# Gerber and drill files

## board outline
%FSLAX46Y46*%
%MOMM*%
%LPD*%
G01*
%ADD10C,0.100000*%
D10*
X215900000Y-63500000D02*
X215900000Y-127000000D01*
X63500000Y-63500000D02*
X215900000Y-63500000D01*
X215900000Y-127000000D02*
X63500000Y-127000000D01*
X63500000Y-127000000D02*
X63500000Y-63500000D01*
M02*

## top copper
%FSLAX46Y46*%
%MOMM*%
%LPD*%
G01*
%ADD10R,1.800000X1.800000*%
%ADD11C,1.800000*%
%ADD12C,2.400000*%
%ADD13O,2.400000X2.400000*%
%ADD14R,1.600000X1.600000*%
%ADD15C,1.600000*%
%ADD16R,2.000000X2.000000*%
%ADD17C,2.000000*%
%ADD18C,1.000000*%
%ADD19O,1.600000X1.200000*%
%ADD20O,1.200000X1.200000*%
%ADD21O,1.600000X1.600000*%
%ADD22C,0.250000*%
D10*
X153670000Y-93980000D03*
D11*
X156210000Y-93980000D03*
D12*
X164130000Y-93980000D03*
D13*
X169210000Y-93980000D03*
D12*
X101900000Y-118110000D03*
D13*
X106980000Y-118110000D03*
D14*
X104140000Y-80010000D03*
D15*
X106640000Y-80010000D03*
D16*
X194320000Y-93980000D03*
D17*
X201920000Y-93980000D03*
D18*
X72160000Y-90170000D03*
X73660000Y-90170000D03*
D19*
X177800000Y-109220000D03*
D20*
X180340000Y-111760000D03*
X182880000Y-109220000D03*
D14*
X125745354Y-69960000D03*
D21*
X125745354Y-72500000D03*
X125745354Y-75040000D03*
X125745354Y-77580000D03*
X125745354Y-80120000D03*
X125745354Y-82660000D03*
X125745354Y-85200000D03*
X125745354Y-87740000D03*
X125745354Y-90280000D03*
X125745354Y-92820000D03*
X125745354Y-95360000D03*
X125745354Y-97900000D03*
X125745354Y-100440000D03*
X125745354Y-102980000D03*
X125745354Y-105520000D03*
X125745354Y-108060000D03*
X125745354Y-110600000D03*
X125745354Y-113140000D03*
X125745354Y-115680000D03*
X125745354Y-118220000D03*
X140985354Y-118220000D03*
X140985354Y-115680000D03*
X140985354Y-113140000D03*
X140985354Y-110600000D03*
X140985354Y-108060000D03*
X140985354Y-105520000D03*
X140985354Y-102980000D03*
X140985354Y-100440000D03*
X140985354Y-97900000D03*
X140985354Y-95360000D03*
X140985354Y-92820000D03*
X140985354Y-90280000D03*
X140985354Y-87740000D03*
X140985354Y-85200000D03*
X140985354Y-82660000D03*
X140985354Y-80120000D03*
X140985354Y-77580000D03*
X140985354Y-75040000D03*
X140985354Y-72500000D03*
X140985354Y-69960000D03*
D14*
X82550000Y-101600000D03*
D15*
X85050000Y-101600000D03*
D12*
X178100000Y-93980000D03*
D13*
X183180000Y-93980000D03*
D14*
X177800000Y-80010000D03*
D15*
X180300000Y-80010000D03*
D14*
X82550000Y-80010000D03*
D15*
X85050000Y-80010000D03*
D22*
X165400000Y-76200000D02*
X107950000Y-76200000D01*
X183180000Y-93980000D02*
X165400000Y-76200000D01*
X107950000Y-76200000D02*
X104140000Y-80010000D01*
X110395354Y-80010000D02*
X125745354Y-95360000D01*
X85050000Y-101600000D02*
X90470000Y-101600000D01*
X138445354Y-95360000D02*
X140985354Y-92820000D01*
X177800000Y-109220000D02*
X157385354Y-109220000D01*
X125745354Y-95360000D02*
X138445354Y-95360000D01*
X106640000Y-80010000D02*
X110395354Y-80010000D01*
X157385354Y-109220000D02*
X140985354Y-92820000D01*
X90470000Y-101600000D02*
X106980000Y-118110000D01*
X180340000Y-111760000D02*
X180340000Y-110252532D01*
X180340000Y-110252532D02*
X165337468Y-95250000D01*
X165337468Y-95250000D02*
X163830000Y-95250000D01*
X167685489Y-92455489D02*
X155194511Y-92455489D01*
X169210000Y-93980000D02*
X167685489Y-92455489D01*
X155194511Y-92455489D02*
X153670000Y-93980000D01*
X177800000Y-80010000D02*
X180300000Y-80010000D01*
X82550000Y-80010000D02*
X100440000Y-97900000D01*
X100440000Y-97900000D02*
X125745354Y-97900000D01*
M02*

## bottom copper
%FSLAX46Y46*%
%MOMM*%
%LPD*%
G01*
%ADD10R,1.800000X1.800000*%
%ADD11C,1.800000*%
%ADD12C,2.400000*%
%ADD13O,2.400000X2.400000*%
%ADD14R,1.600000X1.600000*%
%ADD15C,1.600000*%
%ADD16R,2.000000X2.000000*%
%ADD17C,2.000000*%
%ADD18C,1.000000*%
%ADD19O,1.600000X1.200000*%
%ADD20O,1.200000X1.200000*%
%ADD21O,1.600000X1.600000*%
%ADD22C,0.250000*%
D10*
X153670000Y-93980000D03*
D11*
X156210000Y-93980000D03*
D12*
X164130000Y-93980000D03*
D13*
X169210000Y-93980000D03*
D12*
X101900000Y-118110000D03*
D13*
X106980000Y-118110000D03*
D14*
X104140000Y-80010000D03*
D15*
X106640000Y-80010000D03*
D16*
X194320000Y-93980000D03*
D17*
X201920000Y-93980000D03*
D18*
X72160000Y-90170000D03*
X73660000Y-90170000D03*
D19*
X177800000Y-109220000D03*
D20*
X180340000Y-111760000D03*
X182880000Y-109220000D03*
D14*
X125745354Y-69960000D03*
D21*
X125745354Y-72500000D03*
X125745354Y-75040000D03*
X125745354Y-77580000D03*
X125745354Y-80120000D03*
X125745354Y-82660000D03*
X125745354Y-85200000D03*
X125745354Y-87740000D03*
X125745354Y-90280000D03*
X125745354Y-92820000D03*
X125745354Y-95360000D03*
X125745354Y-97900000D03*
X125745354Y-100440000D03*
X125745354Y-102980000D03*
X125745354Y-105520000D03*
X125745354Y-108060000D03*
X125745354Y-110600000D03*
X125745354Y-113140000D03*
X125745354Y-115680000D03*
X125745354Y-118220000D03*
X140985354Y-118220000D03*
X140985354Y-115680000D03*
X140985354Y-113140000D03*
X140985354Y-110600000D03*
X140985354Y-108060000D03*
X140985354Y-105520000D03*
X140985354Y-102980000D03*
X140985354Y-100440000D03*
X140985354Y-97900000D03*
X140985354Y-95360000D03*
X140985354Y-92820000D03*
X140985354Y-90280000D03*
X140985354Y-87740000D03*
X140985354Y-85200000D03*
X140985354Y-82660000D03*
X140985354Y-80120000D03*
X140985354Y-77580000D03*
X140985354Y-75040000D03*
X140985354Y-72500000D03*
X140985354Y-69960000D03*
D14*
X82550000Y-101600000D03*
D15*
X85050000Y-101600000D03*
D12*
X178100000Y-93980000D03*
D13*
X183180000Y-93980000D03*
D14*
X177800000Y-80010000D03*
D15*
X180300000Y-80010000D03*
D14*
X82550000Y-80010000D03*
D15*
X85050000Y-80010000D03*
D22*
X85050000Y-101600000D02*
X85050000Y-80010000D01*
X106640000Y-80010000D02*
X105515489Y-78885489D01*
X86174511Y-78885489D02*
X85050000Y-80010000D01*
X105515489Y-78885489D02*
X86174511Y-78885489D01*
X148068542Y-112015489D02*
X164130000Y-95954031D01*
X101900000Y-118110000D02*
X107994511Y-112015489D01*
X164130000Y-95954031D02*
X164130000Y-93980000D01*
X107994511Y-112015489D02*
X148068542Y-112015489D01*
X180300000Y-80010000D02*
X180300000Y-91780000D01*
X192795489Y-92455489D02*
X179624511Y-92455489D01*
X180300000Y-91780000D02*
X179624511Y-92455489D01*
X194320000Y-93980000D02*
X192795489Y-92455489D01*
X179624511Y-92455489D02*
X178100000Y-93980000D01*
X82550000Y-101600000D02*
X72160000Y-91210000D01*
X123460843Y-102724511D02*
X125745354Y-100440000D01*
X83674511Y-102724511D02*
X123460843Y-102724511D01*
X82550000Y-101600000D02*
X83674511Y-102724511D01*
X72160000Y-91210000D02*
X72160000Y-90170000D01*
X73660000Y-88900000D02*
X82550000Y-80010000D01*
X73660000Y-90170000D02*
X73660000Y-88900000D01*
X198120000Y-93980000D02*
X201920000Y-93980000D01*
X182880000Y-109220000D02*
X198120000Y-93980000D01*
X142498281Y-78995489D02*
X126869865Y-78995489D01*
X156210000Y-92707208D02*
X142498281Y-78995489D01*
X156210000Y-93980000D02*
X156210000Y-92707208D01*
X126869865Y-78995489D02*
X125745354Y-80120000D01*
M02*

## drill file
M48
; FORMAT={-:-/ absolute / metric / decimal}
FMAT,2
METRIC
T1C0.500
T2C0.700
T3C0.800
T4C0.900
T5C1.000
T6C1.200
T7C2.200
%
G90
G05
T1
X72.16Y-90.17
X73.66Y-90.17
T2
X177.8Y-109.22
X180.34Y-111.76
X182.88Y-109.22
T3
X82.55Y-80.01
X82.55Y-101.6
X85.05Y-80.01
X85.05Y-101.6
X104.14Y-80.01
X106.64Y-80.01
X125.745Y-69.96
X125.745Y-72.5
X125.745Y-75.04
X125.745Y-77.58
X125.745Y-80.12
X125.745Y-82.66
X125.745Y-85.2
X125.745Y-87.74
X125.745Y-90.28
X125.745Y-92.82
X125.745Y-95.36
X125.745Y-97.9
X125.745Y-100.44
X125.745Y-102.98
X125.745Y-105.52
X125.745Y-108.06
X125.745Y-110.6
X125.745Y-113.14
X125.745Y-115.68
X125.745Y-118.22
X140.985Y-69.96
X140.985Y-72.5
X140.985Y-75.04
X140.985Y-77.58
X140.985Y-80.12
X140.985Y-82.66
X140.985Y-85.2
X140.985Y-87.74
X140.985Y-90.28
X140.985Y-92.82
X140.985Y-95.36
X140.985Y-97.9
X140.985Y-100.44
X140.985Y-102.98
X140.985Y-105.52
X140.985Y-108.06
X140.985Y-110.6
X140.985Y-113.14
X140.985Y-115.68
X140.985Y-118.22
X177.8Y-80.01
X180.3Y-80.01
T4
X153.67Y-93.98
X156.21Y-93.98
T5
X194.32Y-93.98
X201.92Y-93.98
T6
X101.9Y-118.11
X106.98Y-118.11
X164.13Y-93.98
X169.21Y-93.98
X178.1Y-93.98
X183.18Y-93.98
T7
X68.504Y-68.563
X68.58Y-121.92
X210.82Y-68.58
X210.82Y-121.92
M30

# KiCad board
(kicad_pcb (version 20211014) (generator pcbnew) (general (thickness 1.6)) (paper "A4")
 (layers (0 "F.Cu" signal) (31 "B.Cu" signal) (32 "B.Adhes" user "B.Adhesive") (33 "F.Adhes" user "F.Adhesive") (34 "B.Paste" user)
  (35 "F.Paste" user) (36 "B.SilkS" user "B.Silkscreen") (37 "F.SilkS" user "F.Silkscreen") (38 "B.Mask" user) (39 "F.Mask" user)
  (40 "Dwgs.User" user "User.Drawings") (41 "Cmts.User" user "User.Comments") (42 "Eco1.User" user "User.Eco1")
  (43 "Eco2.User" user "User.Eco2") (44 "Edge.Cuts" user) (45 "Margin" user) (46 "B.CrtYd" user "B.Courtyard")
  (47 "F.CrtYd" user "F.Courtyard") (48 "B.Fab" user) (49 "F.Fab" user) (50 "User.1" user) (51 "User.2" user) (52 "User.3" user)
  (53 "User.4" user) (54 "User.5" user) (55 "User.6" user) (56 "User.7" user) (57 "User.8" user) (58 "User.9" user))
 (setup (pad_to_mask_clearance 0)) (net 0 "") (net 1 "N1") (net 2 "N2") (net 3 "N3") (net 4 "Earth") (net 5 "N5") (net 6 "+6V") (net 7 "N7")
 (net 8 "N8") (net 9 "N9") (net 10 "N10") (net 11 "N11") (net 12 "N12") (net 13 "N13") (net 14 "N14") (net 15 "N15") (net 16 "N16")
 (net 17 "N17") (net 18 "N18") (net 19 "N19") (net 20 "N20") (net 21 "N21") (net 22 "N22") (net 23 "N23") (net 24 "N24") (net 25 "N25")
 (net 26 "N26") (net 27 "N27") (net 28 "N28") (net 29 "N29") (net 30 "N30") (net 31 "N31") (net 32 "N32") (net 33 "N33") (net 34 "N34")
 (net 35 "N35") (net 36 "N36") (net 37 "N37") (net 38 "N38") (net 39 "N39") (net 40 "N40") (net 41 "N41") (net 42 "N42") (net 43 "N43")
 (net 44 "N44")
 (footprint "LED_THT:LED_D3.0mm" (layer "F.Cu") (at 153.67 93.98)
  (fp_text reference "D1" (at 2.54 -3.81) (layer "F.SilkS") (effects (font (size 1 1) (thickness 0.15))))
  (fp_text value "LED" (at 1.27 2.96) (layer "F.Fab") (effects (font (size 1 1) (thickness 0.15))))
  (pad "1" thru_hole rect (at 0 0) (size 1.8 1.8) (drill 0.9) (layers *.Cu *.Mask) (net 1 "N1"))
  (pad "2" thru_hole circle (at 2.54 0) (size 1.8 1.8) (drill 0.9) (layers *.Cu *.Mask) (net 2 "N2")))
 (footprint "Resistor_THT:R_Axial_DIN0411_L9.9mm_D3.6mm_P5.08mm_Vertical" (layer "F.Cu") (at 164.13 93.98)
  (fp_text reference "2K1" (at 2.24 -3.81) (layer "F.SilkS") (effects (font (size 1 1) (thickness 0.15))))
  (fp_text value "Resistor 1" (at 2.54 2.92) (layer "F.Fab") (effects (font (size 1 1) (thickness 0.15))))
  (pad "1" thru_hole circle (at 0 0) (size 2.4 2.4) (drill 1.2) (layers *.Cu *.Mask) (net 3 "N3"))
  (pad "2" thru_hole oval (at 5.08 0) (size 2.4 2.4) (drill 1.2) (layers *.Cu *.Mask) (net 1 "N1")))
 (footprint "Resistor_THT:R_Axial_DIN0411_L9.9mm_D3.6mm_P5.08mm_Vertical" (layer "F.Cu") (at 101.9 118.11)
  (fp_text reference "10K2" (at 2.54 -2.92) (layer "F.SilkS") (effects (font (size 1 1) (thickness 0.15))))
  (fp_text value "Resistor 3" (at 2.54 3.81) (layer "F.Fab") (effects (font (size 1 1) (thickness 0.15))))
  (pad "1" thru_hole circle (at 0 0) (size 2.4 2.4) (drill 1.2) (layers *.Cu *.Mask) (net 3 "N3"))
  (pad "2" thru_hole oval (at 5.08 0) (size 2.4 2.4) (drill 1.2) (layers *.Cu *.Mask) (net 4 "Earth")))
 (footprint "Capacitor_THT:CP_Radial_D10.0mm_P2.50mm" (layer "F.Cu") (at 104.14 80.01)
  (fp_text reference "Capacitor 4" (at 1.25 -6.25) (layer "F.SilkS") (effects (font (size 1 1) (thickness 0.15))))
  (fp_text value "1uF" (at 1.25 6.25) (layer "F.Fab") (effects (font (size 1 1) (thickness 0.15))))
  (pad "1" thru_hole rect (at 0 0) (size 1.6 1.6) (drill 0.8) (layers *.Cu *.Mask) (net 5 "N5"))
  (pad "2" thru_hole circle (at 2.5 0) (size 1.6 1.6) (drill 0.8) (layers *.Cu *.Mask) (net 4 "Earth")))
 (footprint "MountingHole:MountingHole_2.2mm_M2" (layer "F.Cu") (at 210.82 121.92)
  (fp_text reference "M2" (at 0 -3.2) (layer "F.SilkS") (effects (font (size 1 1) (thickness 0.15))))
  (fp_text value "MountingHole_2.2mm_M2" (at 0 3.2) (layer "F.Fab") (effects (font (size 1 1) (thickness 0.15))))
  (pad "" np_thru_hole circle (at 0 0) (size 2.2 2.2) (drill 2.2) (layers *.Cu *.Mask)))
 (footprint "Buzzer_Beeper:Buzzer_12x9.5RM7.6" (layer "F.Cu") (at 194.32 93.98)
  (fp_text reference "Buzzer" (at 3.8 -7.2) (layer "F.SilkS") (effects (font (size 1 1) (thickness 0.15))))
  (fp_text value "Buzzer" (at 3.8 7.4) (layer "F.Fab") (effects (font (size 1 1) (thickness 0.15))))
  (pad "1" thru_hole rect (at 0 0) (size 2 2) (drill 1) (layers *.Cu *.Mask) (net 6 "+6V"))
  (pad "2" thru_hole circle (at 7.6 0) (size 2 2) (drill 1) (layers *.Cu *.Mask) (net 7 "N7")))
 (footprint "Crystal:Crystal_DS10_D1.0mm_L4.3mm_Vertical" (layer "F.Cu") (at 72.16 90.17)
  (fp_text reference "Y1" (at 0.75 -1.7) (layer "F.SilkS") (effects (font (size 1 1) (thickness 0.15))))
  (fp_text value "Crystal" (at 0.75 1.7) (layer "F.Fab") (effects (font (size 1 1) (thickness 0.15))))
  (pad "1" thru_hole circle (at 0 0) (size 1 1) (drill 0.5) (layers *.Cu *.Mask) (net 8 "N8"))
  (pad "2" thru_hole circle (at 1.5 0) (size 1 1) (drill 0.5) (layers *.Cu *.Mask) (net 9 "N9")))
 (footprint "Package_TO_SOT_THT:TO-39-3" (layer "F.Cu") (at 177.8 109.22)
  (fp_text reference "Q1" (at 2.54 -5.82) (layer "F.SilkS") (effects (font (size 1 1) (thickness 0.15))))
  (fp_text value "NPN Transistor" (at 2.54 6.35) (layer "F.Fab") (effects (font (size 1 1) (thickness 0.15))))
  (pad "1" thru_hole oval (at 0 0) (size 1.6 1.2) (drill 0.7) (layers *.Cu *.Mask) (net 4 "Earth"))
  (pad "2" thru_hole oval (at 2.54 2.54) (size 1.2 1.2) (drill 0.7) (layers *.Cu *.Mask) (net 3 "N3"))
  (pad "3" thru_hole oval (at 5.08 0) (size 1.2 1.2) (drill 0.7) (layers *.Cu *.Mask) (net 7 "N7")))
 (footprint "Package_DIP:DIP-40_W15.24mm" (layer "F.Cu") (at 125.745354 69.96)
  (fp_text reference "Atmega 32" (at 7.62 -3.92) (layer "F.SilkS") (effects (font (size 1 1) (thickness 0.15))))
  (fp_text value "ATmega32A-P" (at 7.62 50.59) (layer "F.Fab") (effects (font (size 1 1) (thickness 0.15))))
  (pad "1" thru_hole rect (at 0 0) (size 1.6 1.6) (drill 0.8) (layers *.Cu *.Mask) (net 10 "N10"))
  (pad "2" thru_hole oval (at 0 2.54) (size 1.6 1.6) (drill 0.8) (layers *.Cu *.Mask) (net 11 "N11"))
  (pad "3" thru_hole oval (at 0 5.08) (size 1.6 1.6) (drill 0.8) (layers *.Cu *.Mask) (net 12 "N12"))
  (pad "4" thru_hole oval (at 0 7.62) (size 1.6 1.6) (drill 0.8) (layers *.Cu *.Mask) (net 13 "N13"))
  (pad "5" thru_hole oval (at 0 10.16) (size 1.6 1.6) (drill 0.8) (layers *.Cu *.Mask) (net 2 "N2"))
  (pad "6" thru_hole oval (at 0 12.7) (size 1.6 1.6) (drill 0.8) (layers *.Cu *.Mask) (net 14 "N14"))
  (pad "7" thru_hole oval (at 0 15.24) (size 1.6 1.6) (drill 0.8) (layers *.Cu *.Mask) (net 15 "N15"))
  (pad "8" thru_hole oval (at 0 17.78) (size 1.6 1.6) (drill 0.8) (layers *.Cu *.Mask) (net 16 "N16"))
  (pad "9" thru_hole oval (at 0 20.32) (size 1.6 1.6) (drill 0.8) (layers *.Cu *.Mask) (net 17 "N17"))
  (pad "10" thru_hole oval (at 0 22.86) (size 1.6 1.6) (drill 0.8) (layers *.Cu *.Mask) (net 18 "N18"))
  (pad "11" thru_hole oval (at 0 25.4) (size 1.6 1.6) (drill 0.8) (layers *.Cu *.Mask) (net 4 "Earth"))
  (pad "12" thru_hole oval (at 0 27.94) (size 1.6 1.6) (drill 0.8) (layers *.Cu *.Mask) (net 9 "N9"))
  (pad "13" thru_hole oval (at 0 30.48) (size 1.6 1.6) (drill 0.8) (layers *.Cu *.Mask) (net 8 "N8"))
  (pad "14" thru_hole oval (at 0 33.02) (size 1.6 1.6) (drill 0.8) (layers *.Cu *.Mask) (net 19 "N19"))
  (pad "15" thru_hole oval (at 0 35.56) (size 1.6 1.6) (drill 0.8) (layers *.Cu *.Mask) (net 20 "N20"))
  (pad "16" thru_hole oval (at 0 38.1) (size 1.6 1.6) (drill 0.8) (layers *.Cu *.Mask) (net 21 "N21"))
  (pad "17" thru_hole oval (at 0 40.64) (size 1.6 1.6) (drill 0.8) (layers *.Cu *.Mask) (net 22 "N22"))
  (pad "18" thru_hole oval (at 0 43.18) (size 1.6 1.6) (drill 0.8) (layers *.Cu *.Mask) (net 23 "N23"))
  (pad "19" thru_hole oval (at 0 45.72) (size 1.6 1.6) (drill 0.8) (layers *.Cu *.Mask) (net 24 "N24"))
  (pad "20" thru_hole oval (at 0 48.26) (size 1.6 1.6) (drill 0.8) (layers *.Cu *.Mask) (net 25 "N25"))
  (pad "21" thru_hole oval (at 15.24 48.26) (size 1.6 1.6) (drill 0.8) (layers *.Cu *.Mask) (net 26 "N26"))
  (pad "22" thru_hole oval (at 15.24 45.72) (size 1.6 1.6) (drill 0.8) (layers *.Cu *.Mask) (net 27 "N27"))
  (pad "23" thru_hole oval (at 15.24 43.18) (size 1.6 1.6) (drill 0.8) (layers *.Cu *.Mask) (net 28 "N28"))
  (pad "24" thru_hole oval (at 15.24 40.64) (size 1.6 1.6) (drill 0.8) (layers *.Cu *.Mask) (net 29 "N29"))
  (pad "25" thru_hole oval (at 15.24 38.1) (size 1.6 1.6) (drill 0.8) (layers *.Cu *.Mask) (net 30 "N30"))
  (pad "26" thru_hole oval (at 15.24 35.56) (size 1.6 1.6) (drill 0.8) (layers *.Cu *.Mask) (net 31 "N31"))
  (pad "27" thru_hole oval (at 15.24 33.02) (size 1.6 1.6) (drill 0.8) (layers *.Cu *.Mask) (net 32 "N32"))
  (pad "28" thru_hole oval (at 15.24 30.48) (size 1.6 1.6) (drill 0.8) (layers *.Cu *.Mask) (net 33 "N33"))
  (pad "29" thru_hole oval (at 15.24 27.94) (size 1.6 1.6) (drill 0.8) (layers *.Cu *.Mask) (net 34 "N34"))
  (pad "30" thru_hole oval (at 15.24 25.4) (size 1.6 1.6) (drill 0.8) (layers *.Cu *.Mask) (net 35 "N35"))
  (pad "31" thru_hole oval (at 15.24 22.86) (size 1.6 1.6) (drill 0.8) (layers *.Cu *.Mask) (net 4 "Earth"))
  (pad "32" thru_hole oval (at 15.24 20.32) (size 1.6 1.6) (drill 0.8) (layers *.Cu *.Mask) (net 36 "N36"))
  (pad "33" thru_hole oval (at 15.24 17.78) (size 1.6 1.6) (drill 0.8) (layers *.Cu *.Mask) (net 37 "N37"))
  (pad "34" thru_hole oval (at 15.24 15.24) (size 1.6 1.6) (drill 0.8) (layers *.Cu *.Mask) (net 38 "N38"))
  (pad "35" thru_hole oval (at 15.24 12.7) (size 1.6 1.6) (drill 0.8) (layers *.Cu *.Mask) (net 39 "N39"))
  (pad "36" thru_hole oval (at 15.24 10.16) (size 1.6 1.6) (drill 0.8) (layers *.Cu *.Mask) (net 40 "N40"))
  (pad "37" thru_hole oval (at 15.24 7.62) (size 1.6 1.6) (drill 0.8) (layers *.Cu *.Mask) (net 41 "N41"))
  (pad "38" thru_hole oval (at 15.24 5.08) (size 1.6 1.6) (drill 0.8) (layers *.Cu *.Mask) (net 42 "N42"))
  (pad "39" thru_hole oval (at 15.24 2.54) (size 1.6 1.6) (drill 0.8) (layers *.Cu *.Mask) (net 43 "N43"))
  (pad "40" thru_hole oval (at 15.24 0) (size 1.6 1.6) (drill 0.8) (layers *.Cu *.Mask) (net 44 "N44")))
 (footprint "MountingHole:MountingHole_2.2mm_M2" (layer "F.Cu") (at 210.82 68.58)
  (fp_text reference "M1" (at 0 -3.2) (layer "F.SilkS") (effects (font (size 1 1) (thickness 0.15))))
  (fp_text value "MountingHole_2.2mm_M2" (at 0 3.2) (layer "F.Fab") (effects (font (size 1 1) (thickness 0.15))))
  (pad "" np_thru_hole circle (at 0 0) (size 2.2 2.2) (drill 2.2) (layers *.Cu *.Mask)))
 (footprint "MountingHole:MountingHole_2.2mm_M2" (layer "F.Cu") (at 68.503658 68.563238)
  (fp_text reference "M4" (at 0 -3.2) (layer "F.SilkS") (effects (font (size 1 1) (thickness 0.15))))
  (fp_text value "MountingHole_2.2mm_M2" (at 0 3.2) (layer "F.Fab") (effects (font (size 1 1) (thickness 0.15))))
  (pad "" np_thru_hole circle (at 0 0) (size 2.2 2.2) (drill 2.2) (layers *.Cu *.Mask)))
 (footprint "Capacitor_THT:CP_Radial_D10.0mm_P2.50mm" (layer "F.Cu") (at 82.55 101.6)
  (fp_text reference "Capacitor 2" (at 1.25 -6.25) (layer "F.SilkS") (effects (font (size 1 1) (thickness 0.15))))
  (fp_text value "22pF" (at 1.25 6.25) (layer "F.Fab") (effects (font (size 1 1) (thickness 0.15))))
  (pad "1" thru_hole rect (at 0 0) (size 1.6 1.6) (drill 0.8) (layers *.Cu *.Mask) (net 8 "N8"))
  (pad "2" thru_hole circle (at 2.5 0) (size 1.6 1.6) (drill 0.8) (layers *.Cu *.Mask) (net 4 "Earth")))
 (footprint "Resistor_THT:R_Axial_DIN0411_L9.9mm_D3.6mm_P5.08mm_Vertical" (layer "F.Cu") (at 178.1 93.98)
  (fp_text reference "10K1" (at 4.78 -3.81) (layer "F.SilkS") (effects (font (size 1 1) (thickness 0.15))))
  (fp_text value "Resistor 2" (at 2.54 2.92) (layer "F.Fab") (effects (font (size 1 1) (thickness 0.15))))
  (pad "1" thru_hole circle (at 0 0) (size 2.4 2.4) (drill 1.2) (layers *.Cu *.Mask) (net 6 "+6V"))
  (pad "2" thru_hole oval (at 5.08 0) (size 2.4 2.4) (drill 1.2) (layers *.Cu *.Mask) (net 5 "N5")))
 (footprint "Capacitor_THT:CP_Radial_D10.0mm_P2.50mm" (layer "F.Cu") (at 177.8 80.01)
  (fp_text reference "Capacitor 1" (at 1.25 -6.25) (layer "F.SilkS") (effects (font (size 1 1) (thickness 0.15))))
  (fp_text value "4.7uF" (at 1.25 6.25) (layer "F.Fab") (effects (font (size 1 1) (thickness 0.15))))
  (pad "1" thru_hole rect (at 0 0) (size 1.6 1.6) (drill 0.8) (layers *.Cu *.Mask) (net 6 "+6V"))
  (pad "2" thru_hole circle (at 2.5 0) (size 1.6 1.6) (drill 0.8) (layers *.Cu *.Mask) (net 6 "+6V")))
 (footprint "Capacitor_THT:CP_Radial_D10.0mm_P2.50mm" (layer "F.Cu") (at 82.55 80.01)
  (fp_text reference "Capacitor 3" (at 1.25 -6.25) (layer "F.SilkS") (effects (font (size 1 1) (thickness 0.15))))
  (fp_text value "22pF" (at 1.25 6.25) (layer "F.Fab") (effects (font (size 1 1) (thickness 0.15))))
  (pad "1" thru_hole rect (at 0 0) (size 1.6 1.6) (drill 0.8) (layers *.Cu *.Mask) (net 9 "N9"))
  (pad "2" thru_hole circle (at 2.5 0) (size 1.6 1.6) (drill 0.8) (layers *.Cu *.Mask) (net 4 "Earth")))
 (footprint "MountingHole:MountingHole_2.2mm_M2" (layer "F.Cu") (at 68.58 121.92)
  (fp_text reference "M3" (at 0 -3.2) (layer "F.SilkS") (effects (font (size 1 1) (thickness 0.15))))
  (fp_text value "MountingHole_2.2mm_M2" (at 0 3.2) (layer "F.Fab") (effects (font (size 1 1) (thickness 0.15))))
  (pad "" np_thru_hole circle (at 0 0) (size 2.2 2.2) (drill 2.2) (layers *.Cu *.Mask)))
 (gr_line (start 215.9 63.5) (end 215.9 127) (layer "Edge.Cuts") (width 0.1))
 (gr_line (start 63.5 63.5) (end 215.9 63.5) (layer "Edge.Cuts") (width 0.1))
 (gr_line (start 215.9 127) (end 63.5 127) (layer "Edge.Cuts") (width 0.1))
 (gr_line (start 63.5 127) (end 63.5 63.5) (layer "Edge.Cuts") (width 0.1))
 (segment (start 165.4 76.2) (end 107.95 76.2) (width 0.25) (layer "F.Cu") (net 5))
 (segment (start 183.18 93.98) (end 165.4 76.2) (width 0.25) (layer "F.Cu") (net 5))
 (segment (start 107.95 76.2) (end 104.14 80.01) (width 0.25) (layer "F.Cu") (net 5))
 (segment (start 110.395354 80.01) (end 125.745354 95.36) (width 0.25) (layer "F.Cu") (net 4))
 (segment (start 85.05 101.6) (end 90.47 101.6) (width 0.25) (layer "F.Cu") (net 4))
 (segment (start 138.445354 95.36) (end 140.985354 92.82) (width 0.25) (layer "F.Cu") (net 4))
 (segment (start 177.8 109.22) (end 157.385354 109.22) (width 0.25) (layer "F.Cu") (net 4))
 (segment (start 125.745354 95.36) (end 138.445354 95.36) (width 0.25) (layer "F.Cu") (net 4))
 (segment (start 106.64 80.01) (end 110.395354 80.01) (width 0.25) (layer "F.Cu") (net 4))
 (segment (start 157.385354 109.22) (end 140.985354 92.82) (width 0.25) (layer "F.Cu") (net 4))
 (segment (start 90.47 101.6) (end 106.98 118.11) (width 0.25) (layer "F.Cu") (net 4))
 (segment (start 85.05 101.6) (end 85.05 80.01) (width 0.25) (layer "B.Cu") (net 4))
 (segment (start 106.64 80.01) (end 105.515489 78.885489) (width 0.25) (layer "B.Cu") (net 4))
 (segment (start 86.174511 78.885489) (end 85.05 80.01) (width 0.25) (layer "B.Cu") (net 4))
 (segment (start 105.515489 78.885489) (end 86.174511 78.885489) (width 0.25) (layer "B.Cu") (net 4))
 (segment (start 180.34 111.76) (end 180.34 110.252532) (width 0.25) (layer "F.Cu") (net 3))
 (segment (start 180.34 110.252532) (end 165.337468 95.25) (width 0.25) (layer "F.Cu") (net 3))
 (segment (start 165.337468 95.25) (end 163.83 95.25) (width 0.25) (layer "F.Cu") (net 3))
 (segment (start 148.068542 112.015489) (end 164.13 95.954031) (width 0.25) (layer "B.Cu") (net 3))
 (segment (start 101.9 118.11) (end 107.994511 112.015489) (width 0.25) (layer "B.Cu") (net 3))
 (segment (start 164.13 95.954031) (end 164.13 93.98) (width 0.25) (layer "B.Cu") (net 3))
 (segment (start 107.994511 112.015489) (end 148.068542 112.015489) (width 0.25) (layer "B.Cu") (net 3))
 (segment (start 167.685489 92.455489) (end 155.194511 92.455489) (width 0.25) (layer "F.Cu") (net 1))
 (segment (start 169.21 93.98) (end 167.685489 92.455489) (width 0.25) (layer "F.Cu") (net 1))
 (segment (start 155.194511 92.455489) (end 153.67 93.98) (width 0.25) (layer "F.Cu") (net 1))
 (segment (start 177.8 80.01) (end 180.3 80.01) (width 0.25) (layer "F.Cu") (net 6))
 (segment (start 180.3 80.01) (end 180.3 91.78) (width 0.25) (layer "B.Cu") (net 6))
 (segment (start 192.795489 92.455489) (end 179.624511 92.455489) (width 0.25) (layer "B.Cu") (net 6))
 (segment (start 180.3 91.78) (end 179.624511 92.455489) (width 0.25) (layer "B.Cu") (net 6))
 (segment (start 194.32 93.98) (end 192.795489 92.455489) (width 0.25) (layer "B.Cu") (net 6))
 (segment (start 179.624511 92.455489) (end 178.1 93.98) (width 0.25) (layer "B.Cu") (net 6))
 (segment (start 82.55 101.6) (end 72.16 91.21) (width 0.25) (layer "B.Cu") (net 8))
 (segment (start 123.460843 102.724511) (end 125.745354 100.44) (width 0.25) (layer "B.Cu") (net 8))
 (segment (start 83.674511 102.724511) (end 123.460843 102.724511) (width 0.25) (layer "B.Cu") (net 8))
 (segment (start 82.55 101.6) (end 83.674511 102.724511) (width 0.25) (layer "B.Cu") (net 8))
 (segment (start 72.16 91.21) (end 72.16 90.17) (width 0.25) (layer "B.Cu") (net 8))
 (segment (start 82.55 80.01) (end 100.44 97.9) (width 0.25) (layer "F.Cu") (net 9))
 (segment (start 100.44 97.9) (end 125.745354 97.9) (width 0.25) (layer "F.Cu") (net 9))
 (segment (start 73.66 88.9) (end 82.55 80.01) (width 0.25) (layer "B.Cu") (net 9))
 (segment (start 73.66 90.17) (end 73.66 88.9) (width 0.25) (layer "B.Cu") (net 9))
 (segment (start 198.12 93.98) (end 201.92 93.98) (width 0.25) (layer "B.Cu") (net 7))
 (segment (start 182.88 109.22) (end 198.12 93.98) (width 0.25) (layer "B.Cu") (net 7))
 (segment (start 142.498281 78.995489) (end 126.869865 78.995489) (width 0.25) (layer "B.Cu") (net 2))
 (segment (start 156.21 92.707208) (end 142.498281 78.995489) (width 0.25) (layer "B.Cu") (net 2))
 (segment (start 156.21 93.98) (end 156.21 92.707208) (width 0.25) (layer "B.Cu") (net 2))
 (segment (start 126.869865 78.995489) (end 125.745354 80.12) (width 0.25) (layer "B.Cu") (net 2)))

